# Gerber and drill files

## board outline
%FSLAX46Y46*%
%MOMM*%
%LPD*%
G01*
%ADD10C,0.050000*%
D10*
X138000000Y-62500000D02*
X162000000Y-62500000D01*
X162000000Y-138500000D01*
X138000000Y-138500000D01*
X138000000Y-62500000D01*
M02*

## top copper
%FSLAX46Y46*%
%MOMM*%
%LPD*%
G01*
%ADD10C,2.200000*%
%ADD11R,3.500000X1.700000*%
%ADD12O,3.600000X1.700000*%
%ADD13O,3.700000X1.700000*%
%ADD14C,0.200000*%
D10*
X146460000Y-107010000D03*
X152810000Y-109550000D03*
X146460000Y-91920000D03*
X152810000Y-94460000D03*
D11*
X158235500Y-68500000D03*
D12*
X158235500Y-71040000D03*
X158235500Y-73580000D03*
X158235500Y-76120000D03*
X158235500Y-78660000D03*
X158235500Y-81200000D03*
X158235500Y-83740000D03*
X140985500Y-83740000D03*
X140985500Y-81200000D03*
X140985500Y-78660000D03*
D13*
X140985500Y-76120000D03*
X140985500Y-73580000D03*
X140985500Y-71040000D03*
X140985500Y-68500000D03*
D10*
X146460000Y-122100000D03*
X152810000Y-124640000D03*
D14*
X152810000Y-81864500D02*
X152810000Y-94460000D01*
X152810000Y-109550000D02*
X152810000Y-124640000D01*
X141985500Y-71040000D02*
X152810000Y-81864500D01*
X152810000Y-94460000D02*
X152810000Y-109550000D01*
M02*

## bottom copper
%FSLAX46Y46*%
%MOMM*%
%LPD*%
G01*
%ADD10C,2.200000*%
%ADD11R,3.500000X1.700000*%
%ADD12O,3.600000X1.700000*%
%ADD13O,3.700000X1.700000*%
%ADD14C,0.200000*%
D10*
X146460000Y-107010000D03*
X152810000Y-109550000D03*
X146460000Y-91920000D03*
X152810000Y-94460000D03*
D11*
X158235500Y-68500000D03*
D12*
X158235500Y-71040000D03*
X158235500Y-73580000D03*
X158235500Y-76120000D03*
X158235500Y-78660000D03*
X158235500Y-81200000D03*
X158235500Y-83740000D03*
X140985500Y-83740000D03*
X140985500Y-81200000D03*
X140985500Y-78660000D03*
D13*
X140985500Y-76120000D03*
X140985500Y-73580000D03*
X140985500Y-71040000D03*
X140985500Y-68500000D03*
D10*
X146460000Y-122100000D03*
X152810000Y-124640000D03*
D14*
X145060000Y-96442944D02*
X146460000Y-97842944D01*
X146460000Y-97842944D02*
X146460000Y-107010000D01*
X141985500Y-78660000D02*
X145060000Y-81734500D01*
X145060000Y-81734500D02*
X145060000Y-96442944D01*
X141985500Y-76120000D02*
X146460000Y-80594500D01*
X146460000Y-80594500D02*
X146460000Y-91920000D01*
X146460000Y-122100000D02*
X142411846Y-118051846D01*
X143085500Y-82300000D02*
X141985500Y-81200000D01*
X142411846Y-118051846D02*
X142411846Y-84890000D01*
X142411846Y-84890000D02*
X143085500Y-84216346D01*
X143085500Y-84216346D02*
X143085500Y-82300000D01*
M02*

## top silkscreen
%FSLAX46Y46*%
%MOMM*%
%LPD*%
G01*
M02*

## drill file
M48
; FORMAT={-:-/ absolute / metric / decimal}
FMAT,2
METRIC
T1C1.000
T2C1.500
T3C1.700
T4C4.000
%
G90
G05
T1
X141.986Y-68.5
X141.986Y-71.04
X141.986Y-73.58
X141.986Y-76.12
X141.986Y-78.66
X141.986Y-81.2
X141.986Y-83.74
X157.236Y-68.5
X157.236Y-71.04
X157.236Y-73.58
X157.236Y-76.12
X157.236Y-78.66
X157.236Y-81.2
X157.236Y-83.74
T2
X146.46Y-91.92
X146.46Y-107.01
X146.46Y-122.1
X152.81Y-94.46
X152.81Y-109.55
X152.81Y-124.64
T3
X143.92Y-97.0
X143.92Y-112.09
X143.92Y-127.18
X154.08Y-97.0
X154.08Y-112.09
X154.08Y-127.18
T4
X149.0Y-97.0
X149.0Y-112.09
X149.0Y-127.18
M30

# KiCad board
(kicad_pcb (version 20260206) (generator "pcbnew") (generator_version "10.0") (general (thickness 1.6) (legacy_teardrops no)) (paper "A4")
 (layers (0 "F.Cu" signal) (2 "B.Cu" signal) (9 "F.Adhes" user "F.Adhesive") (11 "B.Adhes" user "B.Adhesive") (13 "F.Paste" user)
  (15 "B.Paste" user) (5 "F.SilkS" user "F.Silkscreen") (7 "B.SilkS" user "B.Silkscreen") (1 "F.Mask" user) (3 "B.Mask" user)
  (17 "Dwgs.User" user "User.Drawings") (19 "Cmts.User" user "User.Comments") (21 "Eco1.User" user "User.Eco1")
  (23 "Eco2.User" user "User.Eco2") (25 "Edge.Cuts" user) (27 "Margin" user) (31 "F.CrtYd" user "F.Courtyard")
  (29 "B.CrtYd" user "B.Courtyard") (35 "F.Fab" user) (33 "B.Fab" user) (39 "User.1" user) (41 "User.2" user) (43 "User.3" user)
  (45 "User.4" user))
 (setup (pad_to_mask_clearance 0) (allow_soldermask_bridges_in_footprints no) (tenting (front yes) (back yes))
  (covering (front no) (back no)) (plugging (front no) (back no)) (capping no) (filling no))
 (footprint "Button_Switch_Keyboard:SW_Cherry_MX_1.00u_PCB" (layer "B.Cu") (at 146.46 107.01 180)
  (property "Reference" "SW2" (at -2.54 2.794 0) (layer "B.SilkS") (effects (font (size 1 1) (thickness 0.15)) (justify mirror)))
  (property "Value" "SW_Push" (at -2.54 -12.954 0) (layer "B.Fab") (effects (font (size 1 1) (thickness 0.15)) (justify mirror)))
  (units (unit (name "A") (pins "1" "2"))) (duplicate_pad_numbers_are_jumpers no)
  (pad "" np_thru_hole circle (at -7.62 -5.08 180) (size 1.7 1.7) (drill 1.7) (layers "*.Cu" "*.Mask"))
  (pad "" np_thru_hole circle (at -2.54 -5.08 180) (size 4 4) (drill 4) (layers "*.Cu" "*.Mask"))
  (pad "" np_thru_hole circle (at 2.54 -5.08 180) (size 1.7 1.7) (drill 1.7) (layers "*.Cu" "*.Mask"))
  (pad "1" thru_hole circle (at 0 0 180) (size 2.2 2.2) (drill 1.5) (layers "*.Cu" "*.Mask") (remove_unused_layers no)
   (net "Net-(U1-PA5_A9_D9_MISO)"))
  (pad "2" thru_hole circle (at -6.35 -2.54 180) (size 2.2 2.2) (drill 1.5) (layers "*.Cu" "*.Mask") (remove_unused_layers no) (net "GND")))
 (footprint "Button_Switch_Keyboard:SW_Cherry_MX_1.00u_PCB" (layer "B.Cu") (at 146.46 91.92 180)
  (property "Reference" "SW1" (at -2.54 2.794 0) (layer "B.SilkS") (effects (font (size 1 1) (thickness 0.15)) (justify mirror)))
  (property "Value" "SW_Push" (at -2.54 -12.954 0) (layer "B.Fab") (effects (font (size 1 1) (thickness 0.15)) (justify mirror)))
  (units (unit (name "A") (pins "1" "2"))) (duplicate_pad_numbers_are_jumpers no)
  (pad "" np_thru_hole circle (at -7.62 -5.08 180) (size 1.7 1.7) (drill 1.7) (layers "*.Cu" "*.Mask"))
  (pad "" np_thru_hole circle (at -2.54 -5.08 180) (size 4 4) (drill 4) (layers "*.Cu" "*.Mask"))
  (pad "" np_thru_hole circle (at 2.54 -5.08 180) (size 1.7 1.7) (drill 1.7) (layers "*.Cu" "*.Mask"))
  (pad "1" thru_hole circle (at 0 0 180) (size 2.2 2.2) (drill 1.5) (layers "*.Cu" "*.Mask") (remove_unused_layers no)
   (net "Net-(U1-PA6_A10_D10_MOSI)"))
  (pad "2" thru_hole circle (at -6.35 -2.54 180) (size 2.2 2.2) (drill 1.5) (layers "*.Cu" "*.Mask") (remove_unused_layers no) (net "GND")))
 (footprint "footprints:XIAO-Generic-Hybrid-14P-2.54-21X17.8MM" (layer "B.Cu") (at 149.6105 76.12 180)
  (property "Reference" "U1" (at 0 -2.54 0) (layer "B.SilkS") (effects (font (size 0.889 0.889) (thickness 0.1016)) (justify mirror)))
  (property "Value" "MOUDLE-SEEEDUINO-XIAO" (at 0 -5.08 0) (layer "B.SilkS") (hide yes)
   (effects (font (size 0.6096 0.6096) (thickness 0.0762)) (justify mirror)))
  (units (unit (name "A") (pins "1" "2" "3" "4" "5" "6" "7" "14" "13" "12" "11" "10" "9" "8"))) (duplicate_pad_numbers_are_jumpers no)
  (pad "1" thru_hole rect (at -7.625 7.62 180) (size 3.5 1.7) (drill 1 (offset -1 0)) (layers "*.Cu" "*.Mask") (remove_unused_layers no)
   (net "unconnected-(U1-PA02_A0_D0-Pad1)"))
  (pad "2" thru_hole oval (at -7.625 5.08 180) (size 3.6 1.7) (drill 1 (offset -1 0)) (layers "*.Cu" "*.Mask") (remove_unused_layers no)
   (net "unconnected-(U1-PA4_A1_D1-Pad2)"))
  (pad "3" thru_hole oval (at -7.625 2.54 180) (size 3.6 1.7) (drill 1 (offset -1 0)) (layers "*.Cu" "*.Mask") (remove_unused_layers no)
   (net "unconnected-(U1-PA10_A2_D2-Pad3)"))
  (pad "4" thru_hole oval (at -7.625 0 180) (size 3.6 1.7) (drill 1 (offset -1 0)) (layers "*.Cu" "*.Mask") (remove_unused_layers no)
   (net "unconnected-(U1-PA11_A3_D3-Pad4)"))
  (pad "5" thru_hole oval (at -7.625 -2.54 180) (size 3.6 1.7) (drill 1 (offset -1 0)) (layers "*.Cu" "*.Mask") (remove_unused_layers no)
   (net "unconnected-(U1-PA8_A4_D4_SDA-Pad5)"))
  (pad "6" thru_hole oval (at -7.625 -5.08) (size 3.6 1.7) (drill 1 (offset 1 0)) (layers "*.Cu" "*.Mask") (remove_unused_layers no)
   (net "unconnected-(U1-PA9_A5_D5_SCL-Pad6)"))
  (pad "7" thru_hole oval (at -7.625 -7.62 180) (size 3.6 1.7) (drill 1 (offset -1 0)) (layers "*.Cu" "*.Mask") (remove_unused_layers no)
   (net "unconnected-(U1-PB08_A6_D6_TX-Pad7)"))
  (pad "8" thru_hole oval (at 7.625 -7.62 180) (size 3.6 1.7) (drill 1 (offset 1 0)) (layers "*.Cu" "*.Mask") (remove_unused_layers no)
   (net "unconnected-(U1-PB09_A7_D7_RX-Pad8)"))
  (pad "9" thru_hole oval (at 7.625 -5.08 180) (size 3.6 1.7) (drill 1 (offset 1 0)) (layers "*.Cu" "*.Mask") (remove_unused_layers no)
   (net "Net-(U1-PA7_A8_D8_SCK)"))
  (pad "10" thru_hole oval (at 7.625 -2.54 180) (size 3.6 1.7) (drill 1 (offset 1 0)) (layers "*.Cu" "*.Mask") (remove_unused_layers no)
   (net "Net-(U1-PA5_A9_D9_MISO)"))
  (pad "11" thru_hole oval (at 7.625 0 180) (size 3.7 1.7) (drill 1 (offset 1 0)) (layers "*.Cu" "*.Mask") (remove_unused_layers no)
   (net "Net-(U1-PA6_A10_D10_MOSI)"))
  (pad "12" thru_hole oval (at 7.625 2.54 180) (size 3.7 1.7) (drill 1 (offset 1 0)) (layers "*.Cu" "*.Mask") (remove_unused_layers no)
   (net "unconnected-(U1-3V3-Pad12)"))
  (pad "13" thru_hole oval (at 7.625 5.08 180) (size 3.7 1.7) (drill 1 (offset 1 0)) (layers "*.Cu" "*.Mask") (remove_unused_layers no)
   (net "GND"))
  (pad "14" thru_hole oval (at 7.625 7.62 180) (size 3.7 1.7) (drill 1 (offset 1 0)) (layers "*.Cu" "*.Mask") (remove_unused_layers no)
   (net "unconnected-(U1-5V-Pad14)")))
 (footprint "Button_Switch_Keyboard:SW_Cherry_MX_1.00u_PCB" (layer "B.Cu") (at 146.46 122.1 180)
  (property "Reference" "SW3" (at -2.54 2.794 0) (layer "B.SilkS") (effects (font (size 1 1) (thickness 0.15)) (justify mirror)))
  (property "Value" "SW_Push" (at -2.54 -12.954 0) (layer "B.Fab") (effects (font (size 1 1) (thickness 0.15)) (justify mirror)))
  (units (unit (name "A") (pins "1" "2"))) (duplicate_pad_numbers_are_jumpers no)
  (pad "" np_thru_hole circle (at -7.62 -5.08 180) (size 1.7 1.7) (drill 1.7) (layers "*.Cu" "*.Mask"))
  (pad "" np_thru_hole circle (at -2.54 -5.08 180) (size 4 4) (drill 4) (layers "*.Cu" "*.Mask"))
  (pad "" np_thru_hole circle (at 2.54 -5.08 180) (size 1.7 1.7) (drill 1.7) (layers "*.Cu" "*.Mask"))
  (pad "1" thru_hole circle (at 0 0 180) (size 2.2 2.2) (drill 1.5) (layers "*.Cu" "*.Mask") (remove_unused_layers no)
   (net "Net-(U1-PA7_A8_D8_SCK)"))
  (pad "2" thru_hole circle (at -6.35 -2.54 180) (size 2.2 2.2) (drill 1.5) (layers "*.Cu" "*.Mask") (remove_unused_layers no) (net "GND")))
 (gr_rect (start 138 62.5) (end 162 138.5) (stroke (width 0.05) (type default)) (fill no) (layer "Edge.Cuts"))
 (segment (start 145.06 96.442944) (end 146.46 97.842944) (width 0.2) (layer "B.Cu") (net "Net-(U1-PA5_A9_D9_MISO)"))
 (segment (start 146.46 97.842944) (end 146.46 107.01) (width 0.2) (layer "B.Cu") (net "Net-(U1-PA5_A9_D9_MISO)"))
 (segment (start 141.9855 78.66) (end 145.06 81.7345) (width 0.2) (layer "B.Cu") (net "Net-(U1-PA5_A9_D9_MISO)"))
 (segment (start 145.06 81.7345) (end 145.06 96.442944) (width 0.2) (layer "B.Cu") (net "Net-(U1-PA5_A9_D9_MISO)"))
 (segment (start 152.81 81.8645) (end 152.81 94.46) (width 0.2) (layer "F.Cu") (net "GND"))
 (segment (start 152.81 109.55) (end 152.81 124.64) (width 0.2) (layer "F.Cu") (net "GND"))
 (segment (start 141.9855 71.04) (end 152.81 81.8645) (width 0.2) (layer "F.Cu") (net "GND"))
 (segment (start 152.81 94.46) (end 152.81 109.55) (width 0.2) (layer "F.Cu") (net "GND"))
 (segment (start 141.9855 76.12) (end 146.46 80.5945) (width 0.2) (layer "B.Cu") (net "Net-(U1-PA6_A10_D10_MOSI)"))
 (segment (start 146.46 80.5945) (end 146.46 91.92) (width 0.2) (layer "B.Cu") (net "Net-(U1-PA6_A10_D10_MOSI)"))
 (segment (start 146.46 122.1) (end 142.411846 118.051846) (width 0.2) (layer "B.Cu") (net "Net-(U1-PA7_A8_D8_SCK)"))
 (segment (start 143.0855 82.3) (end 141.9855 81.2) (width 0.2) (layer "B.Cu") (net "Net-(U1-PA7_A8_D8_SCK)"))
 (segment (start 142.411846 118.051846) (end 142.411846 84.89) (width 0.2) (layer "B.Cu") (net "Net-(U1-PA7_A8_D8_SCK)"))
 (segment (start 142.411846 84.89) (end 143.0855 84.216346) (width 0.2) (layer "B.Cu") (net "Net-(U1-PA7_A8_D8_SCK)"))
 (segment (start 143.0855 84.216346) (end 143.0855 82.3) (width 0.2) (layer "B.Cu") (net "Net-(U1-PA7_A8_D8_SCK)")))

